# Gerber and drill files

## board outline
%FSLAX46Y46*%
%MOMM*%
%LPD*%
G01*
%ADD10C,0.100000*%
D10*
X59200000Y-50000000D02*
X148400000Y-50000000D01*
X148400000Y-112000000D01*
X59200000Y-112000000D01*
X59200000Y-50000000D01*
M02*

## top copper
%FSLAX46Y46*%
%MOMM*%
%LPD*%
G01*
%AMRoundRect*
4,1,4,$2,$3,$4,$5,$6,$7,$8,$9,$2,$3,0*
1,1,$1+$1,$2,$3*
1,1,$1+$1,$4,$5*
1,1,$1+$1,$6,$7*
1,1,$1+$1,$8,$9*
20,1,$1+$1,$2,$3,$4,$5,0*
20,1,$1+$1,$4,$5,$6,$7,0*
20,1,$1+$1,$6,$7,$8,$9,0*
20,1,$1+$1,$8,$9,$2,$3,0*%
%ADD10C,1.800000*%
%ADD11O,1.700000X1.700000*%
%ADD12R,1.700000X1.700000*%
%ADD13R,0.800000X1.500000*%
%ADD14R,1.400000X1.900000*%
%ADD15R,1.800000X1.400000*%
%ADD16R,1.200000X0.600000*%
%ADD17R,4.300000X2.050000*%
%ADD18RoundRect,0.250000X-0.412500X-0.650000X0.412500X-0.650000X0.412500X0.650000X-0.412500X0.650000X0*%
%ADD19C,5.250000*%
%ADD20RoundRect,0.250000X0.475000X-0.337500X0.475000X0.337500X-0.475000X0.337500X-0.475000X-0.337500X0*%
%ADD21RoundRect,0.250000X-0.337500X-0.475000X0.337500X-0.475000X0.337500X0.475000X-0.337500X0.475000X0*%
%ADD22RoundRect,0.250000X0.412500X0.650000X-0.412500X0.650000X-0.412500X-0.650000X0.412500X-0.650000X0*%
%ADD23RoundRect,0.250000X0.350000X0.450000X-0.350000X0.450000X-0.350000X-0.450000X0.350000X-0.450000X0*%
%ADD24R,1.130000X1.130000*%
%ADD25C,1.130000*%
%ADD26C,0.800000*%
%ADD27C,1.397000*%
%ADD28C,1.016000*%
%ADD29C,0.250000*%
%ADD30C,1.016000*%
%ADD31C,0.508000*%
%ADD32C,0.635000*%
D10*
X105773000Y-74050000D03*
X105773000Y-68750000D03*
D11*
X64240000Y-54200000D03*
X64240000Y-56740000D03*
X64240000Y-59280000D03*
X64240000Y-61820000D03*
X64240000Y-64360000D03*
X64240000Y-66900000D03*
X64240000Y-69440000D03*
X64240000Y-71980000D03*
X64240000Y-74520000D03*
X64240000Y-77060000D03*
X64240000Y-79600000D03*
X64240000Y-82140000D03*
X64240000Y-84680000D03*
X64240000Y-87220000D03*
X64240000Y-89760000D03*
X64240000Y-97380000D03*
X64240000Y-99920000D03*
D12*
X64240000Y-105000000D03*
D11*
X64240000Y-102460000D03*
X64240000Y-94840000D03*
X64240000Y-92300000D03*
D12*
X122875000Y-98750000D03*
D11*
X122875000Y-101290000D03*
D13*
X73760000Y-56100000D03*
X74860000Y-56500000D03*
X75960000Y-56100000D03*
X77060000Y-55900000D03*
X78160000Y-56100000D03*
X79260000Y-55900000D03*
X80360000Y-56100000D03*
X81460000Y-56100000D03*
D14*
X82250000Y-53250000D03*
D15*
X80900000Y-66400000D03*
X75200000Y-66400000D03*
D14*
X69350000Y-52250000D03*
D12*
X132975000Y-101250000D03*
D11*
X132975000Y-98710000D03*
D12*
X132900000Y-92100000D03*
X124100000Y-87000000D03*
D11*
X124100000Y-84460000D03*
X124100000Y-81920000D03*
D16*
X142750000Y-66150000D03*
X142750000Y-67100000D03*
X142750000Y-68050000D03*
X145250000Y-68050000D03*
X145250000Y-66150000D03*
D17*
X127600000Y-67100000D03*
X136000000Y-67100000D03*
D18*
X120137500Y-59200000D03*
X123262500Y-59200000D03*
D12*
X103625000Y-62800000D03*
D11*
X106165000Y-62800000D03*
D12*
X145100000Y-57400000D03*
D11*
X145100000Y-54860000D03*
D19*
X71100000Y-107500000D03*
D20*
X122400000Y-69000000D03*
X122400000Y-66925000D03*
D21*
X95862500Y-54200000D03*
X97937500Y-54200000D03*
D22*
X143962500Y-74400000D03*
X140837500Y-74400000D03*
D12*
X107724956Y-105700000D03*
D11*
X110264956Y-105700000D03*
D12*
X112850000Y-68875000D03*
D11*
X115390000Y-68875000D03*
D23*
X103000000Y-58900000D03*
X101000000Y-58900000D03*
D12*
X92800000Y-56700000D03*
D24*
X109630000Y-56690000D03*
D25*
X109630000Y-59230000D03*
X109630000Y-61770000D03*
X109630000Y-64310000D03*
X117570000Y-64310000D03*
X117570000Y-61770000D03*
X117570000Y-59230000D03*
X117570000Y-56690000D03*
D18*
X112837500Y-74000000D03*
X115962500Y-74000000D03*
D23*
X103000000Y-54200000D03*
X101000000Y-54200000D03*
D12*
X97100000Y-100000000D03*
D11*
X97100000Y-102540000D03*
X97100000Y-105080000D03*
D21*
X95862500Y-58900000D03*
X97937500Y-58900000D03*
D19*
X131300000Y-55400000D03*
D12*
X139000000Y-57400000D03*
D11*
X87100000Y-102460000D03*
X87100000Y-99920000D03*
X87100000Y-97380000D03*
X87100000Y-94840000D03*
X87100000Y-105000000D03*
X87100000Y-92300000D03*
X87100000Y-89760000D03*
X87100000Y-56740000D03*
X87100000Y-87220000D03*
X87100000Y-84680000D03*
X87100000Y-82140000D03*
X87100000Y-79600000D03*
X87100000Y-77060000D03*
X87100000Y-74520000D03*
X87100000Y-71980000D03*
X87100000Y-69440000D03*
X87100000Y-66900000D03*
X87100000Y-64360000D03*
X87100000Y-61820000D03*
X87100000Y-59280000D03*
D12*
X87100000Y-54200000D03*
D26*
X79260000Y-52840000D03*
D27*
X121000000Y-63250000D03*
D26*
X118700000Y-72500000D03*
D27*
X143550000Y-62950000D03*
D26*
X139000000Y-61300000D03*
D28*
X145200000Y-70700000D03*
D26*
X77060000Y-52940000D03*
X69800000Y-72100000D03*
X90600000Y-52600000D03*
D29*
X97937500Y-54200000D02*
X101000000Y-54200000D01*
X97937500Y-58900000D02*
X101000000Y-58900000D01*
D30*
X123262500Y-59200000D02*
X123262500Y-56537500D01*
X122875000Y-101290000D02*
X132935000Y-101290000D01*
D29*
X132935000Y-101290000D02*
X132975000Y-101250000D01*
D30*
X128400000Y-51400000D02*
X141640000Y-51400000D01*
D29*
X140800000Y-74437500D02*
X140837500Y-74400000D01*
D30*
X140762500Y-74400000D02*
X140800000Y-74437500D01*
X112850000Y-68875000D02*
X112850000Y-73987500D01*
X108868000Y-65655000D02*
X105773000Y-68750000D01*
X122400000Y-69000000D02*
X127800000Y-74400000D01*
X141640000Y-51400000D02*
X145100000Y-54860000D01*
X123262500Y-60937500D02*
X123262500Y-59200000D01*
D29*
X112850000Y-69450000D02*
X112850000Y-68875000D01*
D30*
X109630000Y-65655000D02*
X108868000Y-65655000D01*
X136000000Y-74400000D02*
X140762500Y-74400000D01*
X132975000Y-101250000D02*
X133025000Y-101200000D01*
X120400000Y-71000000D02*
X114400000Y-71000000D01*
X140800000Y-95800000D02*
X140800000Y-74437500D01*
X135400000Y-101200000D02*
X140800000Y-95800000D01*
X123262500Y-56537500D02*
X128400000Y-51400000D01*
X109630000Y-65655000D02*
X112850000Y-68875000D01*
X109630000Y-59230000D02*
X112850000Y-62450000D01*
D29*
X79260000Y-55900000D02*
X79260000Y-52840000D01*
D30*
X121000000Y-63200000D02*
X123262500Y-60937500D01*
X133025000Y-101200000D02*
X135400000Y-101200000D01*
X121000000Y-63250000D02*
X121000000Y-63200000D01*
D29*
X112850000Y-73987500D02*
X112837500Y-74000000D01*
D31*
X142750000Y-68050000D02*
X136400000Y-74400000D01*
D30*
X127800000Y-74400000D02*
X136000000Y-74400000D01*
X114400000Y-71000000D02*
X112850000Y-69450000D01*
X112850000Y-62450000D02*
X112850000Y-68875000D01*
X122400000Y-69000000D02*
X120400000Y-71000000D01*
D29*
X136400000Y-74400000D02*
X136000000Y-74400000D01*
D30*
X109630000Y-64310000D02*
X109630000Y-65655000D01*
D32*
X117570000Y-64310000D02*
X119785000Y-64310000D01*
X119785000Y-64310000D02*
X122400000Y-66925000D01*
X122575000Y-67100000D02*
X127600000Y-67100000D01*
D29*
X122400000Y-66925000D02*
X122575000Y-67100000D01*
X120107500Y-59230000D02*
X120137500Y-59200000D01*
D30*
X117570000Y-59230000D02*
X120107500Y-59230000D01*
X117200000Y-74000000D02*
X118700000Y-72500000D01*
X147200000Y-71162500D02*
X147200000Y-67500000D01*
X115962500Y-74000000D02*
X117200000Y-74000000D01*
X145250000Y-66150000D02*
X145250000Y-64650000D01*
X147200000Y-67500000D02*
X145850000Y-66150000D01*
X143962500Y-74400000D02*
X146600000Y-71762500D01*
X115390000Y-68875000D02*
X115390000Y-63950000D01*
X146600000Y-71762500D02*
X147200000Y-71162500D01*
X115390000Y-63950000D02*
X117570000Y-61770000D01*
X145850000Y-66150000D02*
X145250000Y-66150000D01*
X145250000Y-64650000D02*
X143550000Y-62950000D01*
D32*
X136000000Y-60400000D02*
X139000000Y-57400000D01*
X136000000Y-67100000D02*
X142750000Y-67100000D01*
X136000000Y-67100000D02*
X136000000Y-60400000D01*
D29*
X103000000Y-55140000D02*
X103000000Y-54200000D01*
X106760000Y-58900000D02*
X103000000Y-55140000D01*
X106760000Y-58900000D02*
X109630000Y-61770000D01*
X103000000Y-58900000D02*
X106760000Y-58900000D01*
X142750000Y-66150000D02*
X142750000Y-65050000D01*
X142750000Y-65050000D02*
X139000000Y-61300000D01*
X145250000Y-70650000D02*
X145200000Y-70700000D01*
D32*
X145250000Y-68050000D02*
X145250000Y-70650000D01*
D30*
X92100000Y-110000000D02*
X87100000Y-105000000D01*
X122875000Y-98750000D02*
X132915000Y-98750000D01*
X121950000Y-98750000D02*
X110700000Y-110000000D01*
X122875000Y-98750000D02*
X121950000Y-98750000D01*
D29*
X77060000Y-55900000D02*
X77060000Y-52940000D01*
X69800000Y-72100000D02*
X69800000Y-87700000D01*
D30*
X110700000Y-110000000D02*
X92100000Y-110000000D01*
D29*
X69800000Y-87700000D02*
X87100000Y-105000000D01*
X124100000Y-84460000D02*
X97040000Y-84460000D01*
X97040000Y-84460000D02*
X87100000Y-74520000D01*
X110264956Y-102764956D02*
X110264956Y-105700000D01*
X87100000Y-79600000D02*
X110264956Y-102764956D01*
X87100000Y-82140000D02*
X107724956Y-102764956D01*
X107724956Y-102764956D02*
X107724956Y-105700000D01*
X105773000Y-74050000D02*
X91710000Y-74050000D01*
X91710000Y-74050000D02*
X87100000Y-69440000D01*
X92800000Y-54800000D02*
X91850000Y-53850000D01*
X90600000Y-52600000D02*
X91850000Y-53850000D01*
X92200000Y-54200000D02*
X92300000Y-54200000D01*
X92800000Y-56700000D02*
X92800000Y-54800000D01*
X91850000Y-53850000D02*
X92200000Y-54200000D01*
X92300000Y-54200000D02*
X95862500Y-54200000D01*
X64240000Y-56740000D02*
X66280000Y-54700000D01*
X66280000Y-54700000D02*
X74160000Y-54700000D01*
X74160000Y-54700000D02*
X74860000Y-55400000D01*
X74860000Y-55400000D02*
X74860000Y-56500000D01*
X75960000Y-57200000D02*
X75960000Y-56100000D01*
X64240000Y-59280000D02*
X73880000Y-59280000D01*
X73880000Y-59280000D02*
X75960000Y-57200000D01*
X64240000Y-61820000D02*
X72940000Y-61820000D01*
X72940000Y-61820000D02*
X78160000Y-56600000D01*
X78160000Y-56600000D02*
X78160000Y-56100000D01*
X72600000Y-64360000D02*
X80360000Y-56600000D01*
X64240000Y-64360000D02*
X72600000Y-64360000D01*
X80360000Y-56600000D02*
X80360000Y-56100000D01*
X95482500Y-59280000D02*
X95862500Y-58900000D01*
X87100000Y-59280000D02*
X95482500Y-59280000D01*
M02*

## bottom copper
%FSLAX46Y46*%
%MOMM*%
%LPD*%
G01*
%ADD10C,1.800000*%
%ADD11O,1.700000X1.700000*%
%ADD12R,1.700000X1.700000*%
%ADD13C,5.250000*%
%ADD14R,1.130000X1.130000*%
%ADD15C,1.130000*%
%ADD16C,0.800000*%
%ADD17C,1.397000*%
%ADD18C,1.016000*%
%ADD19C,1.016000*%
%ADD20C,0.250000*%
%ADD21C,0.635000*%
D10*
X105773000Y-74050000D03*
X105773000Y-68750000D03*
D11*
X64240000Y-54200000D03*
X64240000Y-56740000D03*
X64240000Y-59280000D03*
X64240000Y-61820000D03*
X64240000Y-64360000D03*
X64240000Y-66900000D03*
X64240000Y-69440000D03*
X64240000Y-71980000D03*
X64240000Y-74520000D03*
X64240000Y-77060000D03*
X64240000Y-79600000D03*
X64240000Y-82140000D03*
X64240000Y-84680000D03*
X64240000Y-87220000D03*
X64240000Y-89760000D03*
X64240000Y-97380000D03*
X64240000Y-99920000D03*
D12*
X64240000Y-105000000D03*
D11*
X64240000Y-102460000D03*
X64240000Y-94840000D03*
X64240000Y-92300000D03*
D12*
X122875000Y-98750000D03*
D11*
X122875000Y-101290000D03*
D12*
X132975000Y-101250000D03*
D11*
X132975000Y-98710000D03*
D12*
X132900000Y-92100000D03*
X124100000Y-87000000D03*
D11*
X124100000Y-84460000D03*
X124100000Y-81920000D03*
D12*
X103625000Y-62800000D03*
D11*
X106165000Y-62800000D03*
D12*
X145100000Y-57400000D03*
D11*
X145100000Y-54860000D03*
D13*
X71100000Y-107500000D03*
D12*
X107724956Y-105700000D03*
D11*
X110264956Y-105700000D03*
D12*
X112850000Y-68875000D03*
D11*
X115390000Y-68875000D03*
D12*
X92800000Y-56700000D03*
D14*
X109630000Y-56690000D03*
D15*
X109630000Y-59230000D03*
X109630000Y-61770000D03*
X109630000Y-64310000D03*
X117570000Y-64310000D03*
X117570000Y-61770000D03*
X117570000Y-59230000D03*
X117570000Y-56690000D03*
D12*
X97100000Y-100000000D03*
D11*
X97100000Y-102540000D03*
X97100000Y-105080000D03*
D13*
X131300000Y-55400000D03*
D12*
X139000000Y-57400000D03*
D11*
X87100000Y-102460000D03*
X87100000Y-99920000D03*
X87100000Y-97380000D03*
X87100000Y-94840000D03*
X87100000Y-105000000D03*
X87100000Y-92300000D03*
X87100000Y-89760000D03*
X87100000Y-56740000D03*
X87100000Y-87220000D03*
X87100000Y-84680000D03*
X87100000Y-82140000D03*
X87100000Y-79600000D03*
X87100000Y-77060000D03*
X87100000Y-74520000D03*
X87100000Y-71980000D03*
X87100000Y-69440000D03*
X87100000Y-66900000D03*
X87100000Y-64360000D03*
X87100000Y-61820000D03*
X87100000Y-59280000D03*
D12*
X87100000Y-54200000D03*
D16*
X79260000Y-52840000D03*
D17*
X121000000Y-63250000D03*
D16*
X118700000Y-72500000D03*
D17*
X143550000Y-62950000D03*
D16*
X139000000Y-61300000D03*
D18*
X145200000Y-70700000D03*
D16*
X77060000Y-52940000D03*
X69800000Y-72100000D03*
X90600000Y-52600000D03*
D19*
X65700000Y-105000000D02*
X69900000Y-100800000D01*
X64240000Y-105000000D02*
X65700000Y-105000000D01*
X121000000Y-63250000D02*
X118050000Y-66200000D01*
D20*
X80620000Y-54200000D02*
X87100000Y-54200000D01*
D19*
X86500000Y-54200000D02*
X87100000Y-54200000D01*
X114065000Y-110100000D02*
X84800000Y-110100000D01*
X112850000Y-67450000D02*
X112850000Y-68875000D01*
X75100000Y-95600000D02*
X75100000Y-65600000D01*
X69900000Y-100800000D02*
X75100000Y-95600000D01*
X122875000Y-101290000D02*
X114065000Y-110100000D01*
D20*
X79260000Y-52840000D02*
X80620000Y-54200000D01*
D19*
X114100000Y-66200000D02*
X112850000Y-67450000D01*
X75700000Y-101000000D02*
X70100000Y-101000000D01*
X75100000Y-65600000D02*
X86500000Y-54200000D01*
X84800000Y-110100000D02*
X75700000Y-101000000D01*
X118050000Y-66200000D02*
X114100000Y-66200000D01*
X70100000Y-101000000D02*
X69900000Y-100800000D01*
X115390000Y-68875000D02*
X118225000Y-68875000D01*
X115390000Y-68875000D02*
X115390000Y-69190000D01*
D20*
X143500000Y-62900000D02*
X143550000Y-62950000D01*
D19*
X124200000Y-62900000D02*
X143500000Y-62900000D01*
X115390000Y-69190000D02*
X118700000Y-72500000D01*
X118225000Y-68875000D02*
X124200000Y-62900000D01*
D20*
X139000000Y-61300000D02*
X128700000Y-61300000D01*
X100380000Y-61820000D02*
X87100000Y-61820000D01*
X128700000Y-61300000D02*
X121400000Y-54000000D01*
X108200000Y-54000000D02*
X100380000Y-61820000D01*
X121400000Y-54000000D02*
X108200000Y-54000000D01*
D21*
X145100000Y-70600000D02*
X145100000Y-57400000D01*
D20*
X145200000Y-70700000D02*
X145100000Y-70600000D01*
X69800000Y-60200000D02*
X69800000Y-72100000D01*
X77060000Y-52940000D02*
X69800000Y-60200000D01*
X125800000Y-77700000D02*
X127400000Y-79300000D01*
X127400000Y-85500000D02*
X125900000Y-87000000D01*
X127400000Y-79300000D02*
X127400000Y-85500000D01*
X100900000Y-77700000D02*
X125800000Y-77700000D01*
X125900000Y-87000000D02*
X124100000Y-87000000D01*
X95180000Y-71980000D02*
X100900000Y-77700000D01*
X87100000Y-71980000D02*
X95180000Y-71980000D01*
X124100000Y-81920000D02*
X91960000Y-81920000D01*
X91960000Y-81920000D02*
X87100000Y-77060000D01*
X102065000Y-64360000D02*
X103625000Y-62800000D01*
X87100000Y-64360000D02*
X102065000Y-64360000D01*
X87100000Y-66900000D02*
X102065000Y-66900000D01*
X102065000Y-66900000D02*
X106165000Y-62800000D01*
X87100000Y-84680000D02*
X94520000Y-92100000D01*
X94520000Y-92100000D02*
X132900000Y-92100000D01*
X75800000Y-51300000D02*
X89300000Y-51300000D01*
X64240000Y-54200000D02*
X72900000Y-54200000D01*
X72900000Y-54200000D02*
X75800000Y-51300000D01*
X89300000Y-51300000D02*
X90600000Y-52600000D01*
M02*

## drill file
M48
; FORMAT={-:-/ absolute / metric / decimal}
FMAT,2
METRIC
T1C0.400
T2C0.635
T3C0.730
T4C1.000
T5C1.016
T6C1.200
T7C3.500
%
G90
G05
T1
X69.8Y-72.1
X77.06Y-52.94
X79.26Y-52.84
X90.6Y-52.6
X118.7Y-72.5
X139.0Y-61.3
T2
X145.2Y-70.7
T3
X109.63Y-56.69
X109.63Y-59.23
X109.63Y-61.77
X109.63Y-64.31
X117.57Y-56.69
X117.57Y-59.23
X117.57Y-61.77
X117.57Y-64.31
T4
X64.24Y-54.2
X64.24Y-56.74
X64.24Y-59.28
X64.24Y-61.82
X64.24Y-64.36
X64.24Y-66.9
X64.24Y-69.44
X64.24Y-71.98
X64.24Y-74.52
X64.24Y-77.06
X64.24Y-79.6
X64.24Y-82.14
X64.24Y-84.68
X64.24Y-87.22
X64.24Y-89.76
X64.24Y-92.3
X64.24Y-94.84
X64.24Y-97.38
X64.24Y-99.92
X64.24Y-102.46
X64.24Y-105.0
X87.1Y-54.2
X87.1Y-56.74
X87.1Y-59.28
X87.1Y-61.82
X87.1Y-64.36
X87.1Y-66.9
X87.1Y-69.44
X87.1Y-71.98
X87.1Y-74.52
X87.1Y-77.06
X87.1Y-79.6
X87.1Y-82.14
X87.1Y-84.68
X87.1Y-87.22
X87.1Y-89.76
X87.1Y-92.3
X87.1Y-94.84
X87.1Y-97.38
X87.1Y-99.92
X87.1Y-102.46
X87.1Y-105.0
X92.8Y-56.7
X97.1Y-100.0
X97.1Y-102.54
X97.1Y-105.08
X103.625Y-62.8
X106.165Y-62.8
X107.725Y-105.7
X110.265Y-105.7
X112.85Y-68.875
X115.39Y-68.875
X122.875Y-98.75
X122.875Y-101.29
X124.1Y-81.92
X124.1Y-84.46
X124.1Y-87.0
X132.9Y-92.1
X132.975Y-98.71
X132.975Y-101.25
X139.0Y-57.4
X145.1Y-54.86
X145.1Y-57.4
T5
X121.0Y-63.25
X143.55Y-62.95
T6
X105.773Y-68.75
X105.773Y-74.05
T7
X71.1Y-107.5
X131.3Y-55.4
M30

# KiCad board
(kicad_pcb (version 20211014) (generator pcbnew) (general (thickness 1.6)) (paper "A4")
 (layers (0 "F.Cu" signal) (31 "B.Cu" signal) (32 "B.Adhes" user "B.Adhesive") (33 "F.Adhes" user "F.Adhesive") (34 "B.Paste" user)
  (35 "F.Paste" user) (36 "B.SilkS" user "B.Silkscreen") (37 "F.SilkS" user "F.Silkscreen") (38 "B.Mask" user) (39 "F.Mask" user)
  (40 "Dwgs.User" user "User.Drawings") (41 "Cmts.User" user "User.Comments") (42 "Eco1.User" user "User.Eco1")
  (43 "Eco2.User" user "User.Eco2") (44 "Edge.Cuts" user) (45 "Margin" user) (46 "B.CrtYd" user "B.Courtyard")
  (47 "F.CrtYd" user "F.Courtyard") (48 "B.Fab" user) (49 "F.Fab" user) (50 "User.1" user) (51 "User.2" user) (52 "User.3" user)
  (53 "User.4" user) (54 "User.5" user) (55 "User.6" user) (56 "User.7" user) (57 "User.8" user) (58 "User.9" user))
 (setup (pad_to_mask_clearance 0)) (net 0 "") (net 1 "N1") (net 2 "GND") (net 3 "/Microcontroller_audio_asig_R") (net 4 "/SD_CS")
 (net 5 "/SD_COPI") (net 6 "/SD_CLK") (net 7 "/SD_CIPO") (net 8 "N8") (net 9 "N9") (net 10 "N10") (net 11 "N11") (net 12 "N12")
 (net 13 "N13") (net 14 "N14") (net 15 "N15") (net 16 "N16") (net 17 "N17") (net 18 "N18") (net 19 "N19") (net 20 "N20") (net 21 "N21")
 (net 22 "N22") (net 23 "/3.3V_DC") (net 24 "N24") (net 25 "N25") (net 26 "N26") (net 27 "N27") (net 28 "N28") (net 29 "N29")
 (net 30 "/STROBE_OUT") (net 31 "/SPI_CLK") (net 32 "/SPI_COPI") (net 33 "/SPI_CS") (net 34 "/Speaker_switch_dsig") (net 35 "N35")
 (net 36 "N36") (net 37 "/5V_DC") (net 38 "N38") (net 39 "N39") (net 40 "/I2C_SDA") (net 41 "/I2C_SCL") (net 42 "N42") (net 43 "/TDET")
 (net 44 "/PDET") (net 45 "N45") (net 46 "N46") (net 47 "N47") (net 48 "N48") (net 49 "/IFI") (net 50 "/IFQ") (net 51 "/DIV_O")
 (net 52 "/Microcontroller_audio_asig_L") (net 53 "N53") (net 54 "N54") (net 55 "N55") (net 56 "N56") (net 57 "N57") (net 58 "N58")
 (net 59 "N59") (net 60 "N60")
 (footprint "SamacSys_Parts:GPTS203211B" (layer "F.Cu") (at 105.854 71.4)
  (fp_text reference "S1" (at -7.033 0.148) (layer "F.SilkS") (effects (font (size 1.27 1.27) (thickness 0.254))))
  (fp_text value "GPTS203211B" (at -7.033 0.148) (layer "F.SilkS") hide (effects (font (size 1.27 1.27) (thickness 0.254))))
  (pad "1" thru_hole circle locked (at -0.081 2.65) (size 1.8 1.8) (drill 1.2) (layers *.Cu *.Mask) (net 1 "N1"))
  (pad "2" thru_hole circle locked (at -0.081 -2.65) (size 1.8 1.8) (drill 1.2) (layers *.Cu *.Mask) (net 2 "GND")))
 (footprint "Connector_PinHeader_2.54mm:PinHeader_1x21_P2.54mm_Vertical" (layer "F.Cu") (at 64.24 105 180)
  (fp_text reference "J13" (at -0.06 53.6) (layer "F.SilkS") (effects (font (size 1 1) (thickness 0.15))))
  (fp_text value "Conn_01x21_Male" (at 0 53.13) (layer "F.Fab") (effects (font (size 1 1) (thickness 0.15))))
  (pad "18" thru_hole oval (at 0 50.8 180) (size 1.7 1.7) (drill 1) (layers *.Cu *.Mask) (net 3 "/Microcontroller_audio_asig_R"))
  (pad "19" thru_hole oval (at 0 48.26 180) (size 1.7 1.7) (drill 1) (layers *.Cu *.Mask) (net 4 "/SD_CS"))
  (pad "20" thru_hole oval (at 0 45.72 180) (size 1.7 1.7) (drill 1) (layers *.Cu *.Mask) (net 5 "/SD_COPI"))
  (pad "21" thru_hole oval (at 0 43.18 180) (size 1.7 1.7) (drill 1) (layers *.Cu *.Mask) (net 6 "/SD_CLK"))
  (pad "26" thru_hole oval (at 0 40.64 180) (size 1.7 1.7) (drill 1) (layers *.Cu *.Mask) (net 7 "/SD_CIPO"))
  (pad "33" thru_hole oval (at 0 38.1 180) (size 1.7 1.7) (drill 1) (layers *.Cu *.Mask) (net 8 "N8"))
  (pad "34" thru_hole oval (at 0 35.56 180) (size 1.7 1.7) (drill 1) (layers *.Cu *.Mask) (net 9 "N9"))
  (pad "35" thru_hole oval (at 0 33.02 180) (size 1.7 1.7) (drill 1) (layers *.Cu *.Mask) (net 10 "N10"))
  (pad "36" thru_hole oval (at 0 30.48 180) (size 1.7 1.7) (drill 1) (layers *.Cu *.Mask) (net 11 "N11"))
  (pad "37" thru_hole oval (at 0 27.94 180) (size 1.7 1.7) (drill 1) (layers *.Cu *.Mask) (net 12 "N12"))
  (pad "38" thru_hole oval (at 0 25.4 180) (size 1.7 1.7) (drill 1) (layers *.Cu *.Mask) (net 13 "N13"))
  (pad "39" thru_hole oval (at 0 22.86 180) (size 1.7 1.7) (drill 1) (layers *.Cu *.Mask) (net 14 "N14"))
  (pad "40" thru_hole oval (at 0 20.32 180) (size 1.7 1.7) (drill 1) (layers *.Cu *.Mask) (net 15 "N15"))
  (pad "41" thru_hole oval (at 0 17.78 180) (size 1.7 1.7) (drill 1) (layers *.Cu *.Mask) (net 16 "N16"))
  (pad "42" thru_hole oval (at 0 15.24 180) (size 1.7 1.7) (drill 1) (layers *.Cu *.Mask) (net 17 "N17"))
  (pad "45" thru_hole oval (at 0 7.62 180) (size 1.7 1.7) (drill 1) (layers *.Cu *.Mask) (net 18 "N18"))
  (pad "46" thru_hole oval (at 0 5.08 180) (size 1.7 1.7) (drill 1) (layers *.Cu *.Mask) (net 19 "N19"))
  (pad "G" thru_hole rect (at 0 0 180) (size 1.7 1.7) (drill 1) (layers *.Cu *.Mask) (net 2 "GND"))
  (pad "RST" thru_hole oval (at 0 2.54 180) (size 1.7 1.7) (drill 1) (layers *.Cu *.Mask) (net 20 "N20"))
  (pad "RX" thru_hole oval (at 0 10.16 180) (size 1.7 1.7) (drill 1) (layers *.Cu *.Mask) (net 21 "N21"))
  (pad "TX" thru_hole oval (at 0 12.7 270) (size 1.7 1.7) (drill 1) (layers *.Cu *.Mask) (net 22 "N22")))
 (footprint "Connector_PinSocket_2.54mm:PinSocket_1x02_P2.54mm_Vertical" (layer "F.Cu") (at 122.875 98.75)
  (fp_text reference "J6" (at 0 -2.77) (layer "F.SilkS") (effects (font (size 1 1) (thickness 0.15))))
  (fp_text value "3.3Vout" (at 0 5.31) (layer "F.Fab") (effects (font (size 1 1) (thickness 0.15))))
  (pad "1" thru_hole rect (at 0 0) (size 1.7 1.7) (drill 1) (layers *.Cu *.Mask) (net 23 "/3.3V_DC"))
  (pad "2" thru_hole oval (at 0 2.54) (size 1.7 1.7) (drill 1) (layers *.Cu *.Mask) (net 2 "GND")))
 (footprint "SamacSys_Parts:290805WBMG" (layer "F.Cu") (at 75.8 59.2)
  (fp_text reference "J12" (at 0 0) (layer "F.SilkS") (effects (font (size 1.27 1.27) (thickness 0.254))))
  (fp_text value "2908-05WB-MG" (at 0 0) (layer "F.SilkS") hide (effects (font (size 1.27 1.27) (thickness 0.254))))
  (pad "1" smd rect locked (at -2.04 -3.1) (size 0.8 1.5) (layers "F.Cu" "F.Paste" "F.Mask") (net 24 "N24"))
  (pad "2" smd rect locked (at -0.94 -2.7) (size 0.8 1.5) (layers "F.Cu" "F.Paste" "F.Mask") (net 4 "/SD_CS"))
  (pad "3" smd rect locked (at 0.16 -3.1) (size 0.8 1.5) (layers "F.Cu" "F.Paste" "F.Mask") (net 5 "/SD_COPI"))
  (pad "4" smd rect locked (at 1.26 -3.3) (size 0.8 1.5) (layers "F.Cu" "F.Paste" "F.Mask") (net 23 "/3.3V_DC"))
  (pad "5" smd rect locked (at 2.36 -3.1) (size 0.8 1.5) (layers "F.Cu" "F.Paste" "F.Mask") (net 6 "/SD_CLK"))
  (pad "6" smd rect locked (at 3.46 -3.3) (size 0.8 1.5) (layers "F.Cu" "F.Paste" "F.Mask") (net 2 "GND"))
  (pad "7" smd rect locked (at 4.56 -3.1) (size 0.8 1.5) (layers "F.Cu" "F.Paste" "F.Mask") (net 7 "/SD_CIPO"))
  (pad "8" smd rect locked (at 5.66 -3.1) (size 0.8 1.5) (layers "F.Cu" "F.Paste" "F.Mask") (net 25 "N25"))
  (pad "MP1" smd rect locked (at 6.45 -5.95) (size 1.4 1.9) (layers "F.Cu" "F.Paste" "F.Mask") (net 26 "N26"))
  (pad "MP2" smd rect locked (at 5.1 7.2 90) (size 1.4 1.8) (layers "F.Cu" "F.Paste" "F.Mask") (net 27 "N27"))
  (pad "MP3" smd rect locked (at -0.6 7.2 90) (size 1.4 1.8) (layers "F.Cu" "F.Paste" "F.Mask") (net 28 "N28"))
  (pad "MP4" smd rect locked (at -6.45 -6.95) (size 1.4 1.9) (layers "F.Cu" "F.Paste" "F.Mask") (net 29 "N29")))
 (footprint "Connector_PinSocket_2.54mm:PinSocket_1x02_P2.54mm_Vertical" (layer "F.Cu") (at 132.975 101.25 180)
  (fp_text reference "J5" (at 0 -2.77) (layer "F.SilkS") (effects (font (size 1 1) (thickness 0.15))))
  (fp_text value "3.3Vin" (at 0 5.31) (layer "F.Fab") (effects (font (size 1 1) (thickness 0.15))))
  (pad "1" thru_hole rect (at 0 0 180) (size 1.7 1.7) (drill 1) (layers *.Cu *.Mask) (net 2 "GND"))
  (pad "2" thru_hole oval (at 0 2.54 180) (size 1.7 1.7) (drill 1) (layers *.Cu *.Mask) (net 23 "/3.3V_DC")))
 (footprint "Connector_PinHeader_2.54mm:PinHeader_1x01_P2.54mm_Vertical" (layer "F.Cu") (at 132.9 92.1)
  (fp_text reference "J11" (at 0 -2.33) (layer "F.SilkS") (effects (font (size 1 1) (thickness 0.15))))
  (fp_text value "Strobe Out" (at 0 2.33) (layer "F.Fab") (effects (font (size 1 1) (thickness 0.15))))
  (pad "1" thru_hole rect (at 0 0) (size 1.7 1.7) (drill 1) (layers *.Cu *.Mask) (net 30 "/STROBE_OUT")))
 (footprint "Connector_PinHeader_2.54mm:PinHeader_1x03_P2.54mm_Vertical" (layer "F.Cu") (at 124.1 87 180)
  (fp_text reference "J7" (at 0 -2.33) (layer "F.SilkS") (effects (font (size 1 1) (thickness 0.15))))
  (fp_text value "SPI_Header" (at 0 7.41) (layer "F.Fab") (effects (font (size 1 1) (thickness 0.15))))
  (pad "1" thru_hole rect (at 0 0 180) (size 1.7 1.7) (drill 1) (layers *.Cu *.Mask) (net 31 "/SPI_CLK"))
  (pad "2" thru_hole oval (at 0 2.54 180) (size 1.7 1.7) (drill 1) (layers *.Cu *.Mask) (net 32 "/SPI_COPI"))
  (pad "3" thru_hole oval (at 0 5.08 180) (size 1.7 1.7) (drill 1) (layers *.Cu *.Mask) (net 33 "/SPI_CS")))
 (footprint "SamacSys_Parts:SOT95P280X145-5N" (layer "F.Cu") (at 144 67.1)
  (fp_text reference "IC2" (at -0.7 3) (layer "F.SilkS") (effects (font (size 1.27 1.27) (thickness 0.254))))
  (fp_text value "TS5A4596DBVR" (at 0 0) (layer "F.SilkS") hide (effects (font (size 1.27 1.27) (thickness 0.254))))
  (pad "1" smd rect locked (at -1.25 -0.95 90) (size 0.6 1.2) (layers "F.Cu" "F.Paste" "F.Mask") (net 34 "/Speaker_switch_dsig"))
  (pad "2" smd rect locked (at -1.25 0 90) (size 0.6 1.2) (layers "F.Cu" "F.Paste" "F.Mask") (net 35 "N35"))
  (pad "3" smd rect locked (at -1.25 0.95 90) (size 0.6 1.2) (layers "F.Cu" "F.Paste" "F.Mask") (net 2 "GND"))
  (pad "4" smd rect locked (at 1.25 0.95 90) (size 0.6 1.2) (layers "F.Cu" "F.Paste" "F.Mask") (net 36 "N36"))
  (pad "5" smd rect locked (at 1.25 -0.95 90) (size 0.6 1.2) (layers "F.Cu" "F.Paste" "F.Mask") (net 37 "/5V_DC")))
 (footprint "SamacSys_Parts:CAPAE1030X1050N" (layer "F.Cu") (at 131.8 67.1)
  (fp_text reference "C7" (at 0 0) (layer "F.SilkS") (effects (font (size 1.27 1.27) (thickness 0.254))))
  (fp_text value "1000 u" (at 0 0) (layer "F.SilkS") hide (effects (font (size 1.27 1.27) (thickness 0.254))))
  (pad "1" smd rect locked (at -4.2 0 90) (size 2.05 4.3) (layers "F.Cu" "F.Paste" "F.Mask") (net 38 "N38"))
  (pad "2" smd rect locked (at 4.2 0 90) (size 2.05 4.3) (layers "F.Cu" "F.Paste" "F.Mask") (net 35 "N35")))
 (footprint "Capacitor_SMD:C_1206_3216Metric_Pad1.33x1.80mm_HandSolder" (layer "F.Cu") (at 121.7 59.2)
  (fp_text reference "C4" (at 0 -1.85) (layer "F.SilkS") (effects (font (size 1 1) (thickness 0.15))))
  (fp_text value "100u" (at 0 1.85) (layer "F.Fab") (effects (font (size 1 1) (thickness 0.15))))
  (pad "1" smd roundrect (at -1.5625 0) (size 1.325 1.8) (layers "F.Cu" "F.Paste" "F.Mask") (roundrect_rratio 0.1886792453) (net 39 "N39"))
  (pad "2" smd roundrect (at 1.5625 0) (size 1.325 1.8) (layers "F.Cu" "F.Paste" "F.Mask") (roundrect_rratio 0.1886792453) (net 2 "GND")))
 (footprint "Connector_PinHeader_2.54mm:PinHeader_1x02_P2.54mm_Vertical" (layer "F.Cu") (at 103.625 62.8 90)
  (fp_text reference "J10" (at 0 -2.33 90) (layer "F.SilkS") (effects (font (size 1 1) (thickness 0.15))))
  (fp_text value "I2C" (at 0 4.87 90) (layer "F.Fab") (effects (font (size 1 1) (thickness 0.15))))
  (pad "1" thru_hole rect (at 0 0 90) (size 1.7 1.7) (drill 1) (layers *.Cu *.Mask) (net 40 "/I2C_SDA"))
  (pad "2" thru_hole oval (at 0 2.54 90) (size 1.7 1.7) (drill 1) (layers *.Cu *.Mask) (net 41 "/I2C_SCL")))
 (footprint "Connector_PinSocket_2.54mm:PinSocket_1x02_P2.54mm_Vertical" (layer "F.Cu") (at 145.1 57.4 180)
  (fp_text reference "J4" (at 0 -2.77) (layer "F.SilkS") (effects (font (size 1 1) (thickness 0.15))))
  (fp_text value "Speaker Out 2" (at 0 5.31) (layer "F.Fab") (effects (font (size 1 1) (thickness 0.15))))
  (pad "1" thru_hole rect (at 0 0 180) (size 1.7 1.7) (drill 1) (layers *.Cu *.Mask) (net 36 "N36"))
  (pad "2" thru_hole oval (at 0 2.54 180) (size 1.7 1.7) (drill 1) (layers *.Cu *.Mask) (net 2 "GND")))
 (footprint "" (layer "F.Cu") (at 71.1 107.5)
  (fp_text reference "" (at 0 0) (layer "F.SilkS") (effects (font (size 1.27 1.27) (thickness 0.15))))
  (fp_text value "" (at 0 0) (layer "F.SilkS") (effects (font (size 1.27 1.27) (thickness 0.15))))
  (pad "MH1" thru_hole circle (at 0 0 90) (size 5.25 5.25) (drill 3.5) (layers *.Cu *.Mask)))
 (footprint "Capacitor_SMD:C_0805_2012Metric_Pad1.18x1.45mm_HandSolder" (layer "F.Cu") (at 122.4 67.9625 90)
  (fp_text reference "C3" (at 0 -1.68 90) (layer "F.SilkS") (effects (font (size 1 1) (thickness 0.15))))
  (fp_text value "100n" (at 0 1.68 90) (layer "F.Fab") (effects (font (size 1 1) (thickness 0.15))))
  (pad "1" smd roundrect (at -1.0375 0 90) (size 1.175 1.45) (layers "F.Cu" "F.Paste" "F.Mask") (roundrect_rratio 0.2127659574)
   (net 2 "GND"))
  (pad "2" smd roundrect (at 1.0375 0 90) (size 1.175 1.45) (layers "F.Cu" "F.Paste" "F.Mask") (roundrect_rratio 0.2127659574)
   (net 38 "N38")))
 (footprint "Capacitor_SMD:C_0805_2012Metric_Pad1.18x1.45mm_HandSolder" (layer "F.Cu") (at 96.9 54.2)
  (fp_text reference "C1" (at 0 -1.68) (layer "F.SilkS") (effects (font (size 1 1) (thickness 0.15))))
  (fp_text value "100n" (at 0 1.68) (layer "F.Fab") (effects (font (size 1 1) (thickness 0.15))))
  (pad "1" smd roundrect (at -1.0375 0) (size 1.175 1.45) (layers "F.Cu" "F.Paste" "F.Mask") (roundrect_rratio 0.2127659574)
   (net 3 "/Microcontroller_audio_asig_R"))
  (pad "2" smd roundrect (at 1.0375 0) (size 1.175 1.45) (layers "F.Cu" "F.Paste" "F.Mask") (roundrect_rratio 0.2127659574) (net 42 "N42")))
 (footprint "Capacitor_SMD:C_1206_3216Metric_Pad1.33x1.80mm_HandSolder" (layer "F.Cu") (at 142.4 74.4 180)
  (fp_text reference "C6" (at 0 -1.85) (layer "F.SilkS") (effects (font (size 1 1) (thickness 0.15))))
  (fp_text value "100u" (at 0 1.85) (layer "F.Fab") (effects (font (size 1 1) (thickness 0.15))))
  (pad "1" smd roundrect (at -1.5625 0 180) (size 1.325 1.8) (layers "F.Cu" "F.Paste" "F.Mask") (roundrect_rratio 0.1886792453)
   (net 37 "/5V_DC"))
  (pad "2" smd roundrect (at 1.5625 0 180) (size 1.325 1.8) (layers "F.Cu" "F.Paste" "F.Mask") (roundrect_rratio 0.1886792453) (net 2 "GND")))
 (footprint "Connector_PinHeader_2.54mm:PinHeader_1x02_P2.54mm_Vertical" (layer "F.Cu") (at 107.724956 105.7 90)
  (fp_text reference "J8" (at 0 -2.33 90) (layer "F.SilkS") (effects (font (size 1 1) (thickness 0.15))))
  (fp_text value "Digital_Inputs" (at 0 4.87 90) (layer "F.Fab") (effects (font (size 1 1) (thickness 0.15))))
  (pad "1" thru_hole rect (at 0 0 90) (size 1.7 1.7) (drill 1) (layers *.Cu *.Mask) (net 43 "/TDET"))
  (pad "2" thru_hole oval (at 0 2.54 90) (size 1.7 1.7) (drill 1) (layers *.Cu *.Mask) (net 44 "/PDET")))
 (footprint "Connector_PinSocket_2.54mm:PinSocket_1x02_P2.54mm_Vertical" (layer "F.Cu") (at 112.85 68.875 90)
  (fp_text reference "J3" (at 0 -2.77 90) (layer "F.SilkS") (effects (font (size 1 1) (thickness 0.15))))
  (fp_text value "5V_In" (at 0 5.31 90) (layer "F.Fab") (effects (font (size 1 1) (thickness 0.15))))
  (pad "1" thru_hole rect (at 0 0 90) (size 1.7 1.7) (drill 1) (layers *.Cu *.Mask) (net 2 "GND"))
  (pad "2" thru_hole oval (at 0 2.54 90) (size 1.7 1.7) (drill 1) (layers *.Cu *.Mask) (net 37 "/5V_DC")))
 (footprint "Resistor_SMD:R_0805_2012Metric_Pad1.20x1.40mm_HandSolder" (layer "F.Cu") (at 102 58.9 180)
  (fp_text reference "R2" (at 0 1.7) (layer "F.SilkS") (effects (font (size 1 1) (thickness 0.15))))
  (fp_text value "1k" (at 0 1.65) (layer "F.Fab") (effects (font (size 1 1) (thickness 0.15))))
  (pad "1" smd roundrect (at -1 0 180) (size 1.2 1.4) (layers "F.Cu" "F.Paste" "F.Mask") (roundrect_rratio 0.2083333333) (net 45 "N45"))
  (pad "2" smd roundrect (at 1 0 180) (size 1.2 1.4) (layers "F.Cu" "F.Paste" "F.Mask") (roundrect_rratio 0.2083333333) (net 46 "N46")))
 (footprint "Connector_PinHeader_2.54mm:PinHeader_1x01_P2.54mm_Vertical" (layer "F.Cu") (at 92.8 56.7)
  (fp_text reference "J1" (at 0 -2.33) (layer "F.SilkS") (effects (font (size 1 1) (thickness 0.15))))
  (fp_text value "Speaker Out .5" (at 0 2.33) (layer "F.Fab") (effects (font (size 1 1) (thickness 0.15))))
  (pad "1" thru_hole rect (at 0 0) (size 1.7 1.7) (drill 1) (layers *.Cu *.Mask) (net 3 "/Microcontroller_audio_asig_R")))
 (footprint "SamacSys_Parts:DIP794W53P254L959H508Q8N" (layer "F.Cu") (at 113.6 60.5)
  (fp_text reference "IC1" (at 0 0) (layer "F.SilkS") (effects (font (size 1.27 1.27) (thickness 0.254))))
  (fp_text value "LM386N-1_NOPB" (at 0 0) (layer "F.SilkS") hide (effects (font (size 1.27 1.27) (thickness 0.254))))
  (pad "1" thru_hole rect locked (at -3.97 -3.81) (size 1.13 1.13) (drill 0.73) (layers *.Cu *.Mask) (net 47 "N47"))
  (pad "2" thru_hole circle locked (at -3.97 -1.27) (size 1.13 1.13) (drill 0.73) (layers *.Cu *.Mask) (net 2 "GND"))
  (pad "3" thru_hole circle locked (at -3.97 1.27) (size 1.13 1.13) (drill 0.73) (layers *.Cu *.Mask) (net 45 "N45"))
  (pad "4" thru_hole circle locked (at -3.97 3.81) (size 1.13 1.13) (drill 0.73) (layers *.Cu *.Mask) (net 2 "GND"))
  (pad "5" thru_hole circle locked (at 3.97 3.81) (size 1.13 1.13) (drill 0.73) (layers *.Cu *.Mask) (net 38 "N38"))
  (pad "6" thru_hole circle locked (at 3.97 1.27) (size 1.13 1.13) (drill 0.73) (layers *.Cu *.Mask) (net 37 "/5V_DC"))
  (pad "7" thru_hole circle locked (at 3.97 -1.27) (size 1.13 1.13) (drill 0.73) (layers *.Cu *.Mask) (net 39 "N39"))
  (pad "8" thru_hole circle locked (at 3.97 -3.81) (size 1.13 1.13) (drill 0.73) (layers *.Cu *.Mask) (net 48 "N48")))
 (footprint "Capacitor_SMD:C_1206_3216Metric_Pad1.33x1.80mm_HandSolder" (layer "F.Cu") (at 114.4 74)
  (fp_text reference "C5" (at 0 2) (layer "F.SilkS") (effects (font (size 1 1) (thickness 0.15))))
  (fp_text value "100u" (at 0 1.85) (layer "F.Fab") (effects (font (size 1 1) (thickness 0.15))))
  (pad "1" smd roundrect (at -1.5625 0) (size 1.325 1.8) (layers "F.Cu" "F.Paste" "F.Mask") (roundrect_rratio 0.1886792453) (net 2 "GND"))
  (pad "2" smd roundrect (at 1.5625 0) (size 1.325 1.8) (layers "F.Cu" "F.Paste" "F.Mask") (roundrect_rratio 0.1886792453) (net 37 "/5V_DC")))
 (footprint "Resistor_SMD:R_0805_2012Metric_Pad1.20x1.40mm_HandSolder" (layer "F.Cu") (at 102 54.2 180)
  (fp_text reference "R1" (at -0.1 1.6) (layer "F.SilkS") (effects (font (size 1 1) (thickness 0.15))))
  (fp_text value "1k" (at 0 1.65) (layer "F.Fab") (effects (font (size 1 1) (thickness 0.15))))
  (pad "1" smd roundrect (at -1 0 180) (size 1.2 1.4) (layers "F.Cu" "F.Paste" "F.Mask") (roundrect_rratio 0.2083333333) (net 45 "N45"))
  (pad "2" smd roundrect (at 1 0 180) (size 1.2 1.4) (layers "F.Cu" "F.Paste" "F.Mask") (roundrect_rratio 0.2083333333) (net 42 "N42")))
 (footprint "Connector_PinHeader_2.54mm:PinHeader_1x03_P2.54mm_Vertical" (layer "F.Cu") (at 97.1 100)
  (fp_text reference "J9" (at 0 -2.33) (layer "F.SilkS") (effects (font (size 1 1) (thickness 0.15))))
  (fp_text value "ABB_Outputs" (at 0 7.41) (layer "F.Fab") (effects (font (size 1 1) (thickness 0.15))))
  (pad "1" thru_hole rect (at 0 0) (size 1.7 1.7) (drill 1) (layers *.Cu *.Mask) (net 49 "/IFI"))
  (pad "2" thru_hole oval (at 0 2.54) (size 1.7 1.7) (drill 1) (layers *.Cu *.Mask) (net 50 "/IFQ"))
  (pad "3" thru_hole oval (at 0 5.08) (size 1.7 1.7) (drill 1) (layers *.Cu *.Mask) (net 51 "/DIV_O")))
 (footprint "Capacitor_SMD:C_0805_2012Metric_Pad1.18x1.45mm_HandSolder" (layer "F.Cu") (at 96.9 58.9)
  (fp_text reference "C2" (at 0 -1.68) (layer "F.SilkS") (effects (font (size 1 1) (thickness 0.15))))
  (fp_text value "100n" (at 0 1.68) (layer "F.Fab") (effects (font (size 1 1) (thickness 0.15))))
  (pad "1" smd roundrect (at -1.0375 0) (size 1.175 1.45) (layers "F.Cu" "F.Paste" "F.Mask") (roundrect_rratio 0.2127659574)
   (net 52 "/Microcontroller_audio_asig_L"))
  (pad "2" smd roundrect (at 1.0375 0) (size 1.175 1.45) (layers "F.Cu" "F.Paste" "F.Mask") (roundrect_rratio 0.2127659574) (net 46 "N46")))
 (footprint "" (layer "F.Cu") (at 131.3 55.4)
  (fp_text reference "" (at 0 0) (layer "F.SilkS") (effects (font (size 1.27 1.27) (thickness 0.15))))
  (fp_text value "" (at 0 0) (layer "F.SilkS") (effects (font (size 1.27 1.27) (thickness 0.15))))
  (pad "MH2" thru_hole circle (at 0 0 90) (size 5.25 5.25) (drill 3.5) (layers *.Cu *.Mask)))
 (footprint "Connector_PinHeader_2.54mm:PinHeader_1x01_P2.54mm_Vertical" (layer "F.Cu") (at 139 57.4)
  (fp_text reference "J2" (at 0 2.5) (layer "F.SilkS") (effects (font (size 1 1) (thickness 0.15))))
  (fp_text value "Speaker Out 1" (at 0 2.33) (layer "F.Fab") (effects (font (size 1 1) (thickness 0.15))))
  (pad "1" thru_hole rect (at 0 0) (size 1.7 1.7) (drill 1) (layers *.Cu *.Mask) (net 35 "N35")))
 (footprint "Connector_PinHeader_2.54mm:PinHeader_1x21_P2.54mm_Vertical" (layer "F.Cu") (at 87.1 54.2)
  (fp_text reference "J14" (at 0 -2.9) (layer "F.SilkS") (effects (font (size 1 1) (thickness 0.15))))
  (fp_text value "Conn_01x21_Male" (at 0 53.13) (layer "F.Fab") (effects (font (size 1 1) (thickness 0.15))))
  (pad "0" thru_hole oval (at 0 48.26) (size 1.7 1.7) (drill 1) (layers *.Cu *.Mask) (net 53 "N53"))
  (pad "1" thru_hole oval (at 0 45.72) (size 1.7 1.7) (drill 1) (layers *.Cu *.Mask) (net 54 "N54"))
  (pad "2" thru_hole oval (at 0 43.18) (size 1.7 1.7) (drill 1) (layers *.Cu *.Mask) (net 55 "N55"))
  (pad "3" thru_hole oval (at 0 40.64) (size 1.7 1.7) (drill 1) (layers *.Cu *.Mask) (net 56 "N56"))
  (pad "3V3" thru_hole oval (at 0 50.8) (size 1.7 1.7) (drill 1) (layers *.Cu *.Mask) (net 23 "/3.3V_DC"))
  (pad "4" thru_hole oval (at 0 38.1) (size 1.7 1.7) (drill 1) (layers *.Cu *.Mask) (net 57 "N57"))
  (pad "5" thru_hole oval (at 0 35.56) (size 1.7 1.7) (drill 1) (layers *.Cu *.Mask) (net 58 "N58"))
  (pad "5V" thru_hole oval (at 0 2.54) (size 1.7 1.7) (drill 1) (layers *.Cu *.Mask) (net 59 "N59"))
  (pad "6" thru_hole oval (at 0 33.02) (size 1.7 1.7) (drill 1) (layers *.Cu *.Mask) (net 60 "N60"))
  (pad "7" thru_hole oval (at 0 30.48) (size 1.7 1.7) (drill 1) (layers *.Cu *.Mask) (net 30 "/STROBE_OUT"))
  (pad "8" thru_hole oval (at 0 27.94) (size 1.7 1.7) (drill 1) (layers *.Cu *.Mask) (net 43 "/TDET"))
  (pad "9" thru_hole oval (at 0 25.4) (size 1.7 1.7) (drill 1) (layers *.Cu *.Mask) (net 44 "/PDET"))
  (pad "10" thru_hole oval (at 0 22.86) (size 1.7 1.7) (drill 1) (layers *.Cu *.Mask) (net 33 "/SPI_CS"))
  (pad "11" thru_hole oval (at 0 20.32) (size 1.7 1.7) (drill 1) (layers *.Cu *.Mask) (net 32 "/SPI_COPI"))
  (pad "12" thru_hole oval (at 0 17.78) (size 1.7 1.7) (drill 1) (layers *.Cu *.Mask) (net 31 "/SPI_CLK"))
  (pad "13" thru_hole oval (at 0 15.24) (size 1.7 1.7) (drill 1) (layers *.Cu *.Mask) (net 1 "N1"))
  (pad "14" thru_hole oval (at 0 12.7) (size 1.7 1.7) (drill 1) (layers *.Cu *.Mask) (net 41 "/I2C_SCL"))
  (pad "15" thru_hole oval (at 0 10.16) (size 1.7 1.7) (drill 1) (layers *.Cu *.Mask) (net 40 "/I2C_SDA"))
  (pad "16" thru_hole oval (at 0 7.62) (size 1.7 1.7) (drill 1) (layers *.Cu *.Mask) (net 34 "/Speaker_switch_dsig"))
  (pad "17" thru_hole oval (at 0 5.08) (size 1.7 1.7) (drill 1) (layers *.Cu *.Mask) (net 52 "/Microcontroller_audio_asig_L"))
  (pad "G" thru_hole rect (at 0 0) (size 1.7 1.7) (drill 1) (layers *.Cu *.Mask) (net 2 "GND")))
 (gr_rect (start 59.2 50) (end 148.4 112) (layer "Edge.Cuts") (width 0.1) (fill none))
 (segment (start 97.9375 54.2) (end 101 54.2) (width 0.25) (layer "F.Cu") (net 42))
 (segment (start 97.9375 58.9) (end 101 58.9) (width 0.25) (layer "F.Cu") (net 46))
 (segment (start 123.2625 59.2) (end 123.2625 56.5375) (width 1.016) (layer "F.Cu") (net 2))
 (segment (start 122.875 101.29) (end 132.935 101.29) (width 1.016) (layer "F.Cu") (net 2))
 (segment (start 132.935 101.29) (end 132.975 101.25) (width 0.25) (layer "F.Cu") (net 2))
 (segment (start 128.4 51.4) (end 141.64 51.4) (width 1.016) (layer "F.Cu") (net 2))
 (segment (start 140.8 74.4375) (end 140.8375 74.4) (width 0.25) (layer "F.Cu") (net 2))
 (segment (start 140.7625 74.4) (end 140.8 74.4375) (width 1.016) (layer "F.Cu") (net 2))
 (segment (start 112.85 68.875) (end 112.85 73.9875) (width 1.016) (layer "F.Cu") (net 2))
 (segment (start 108.868 65.655) (end 105.773 68.75) (width 1.016) (layer "F.Cu") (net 2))
 (segment (start 122.4 69) (end 127.8 74.4) (width 1.016) (layer "F.Cu") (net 2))
 (segment (start 141.64 51.4) (end 145.1 54.86) (width 1.016) (layer "F.Cu") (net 2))
 (segment (start 123.2625 60.9375) (end 123.2625 59.2) (width 1.016) (layer "F.Cu") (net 2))
 (segment (start 112.85 69.45) (end 112.85 68.875) (width 0.25) (layer "F.Cu") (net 2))
 (segment (start 109.63 65.655) (end 108.868 65.655) (width 1.016) (layer "F.Cu") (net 2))
 (segment (start 136 74.4) (end 140.7625 74.4) (width 1.016) (layer "F.Cu") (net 2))
 (segment (start 132.975 101.25) (end 133.025 101.2) (width 1.016) (layer "F.Cu") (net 2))
 (segment (start 120.4 71) (end 114.4 71) (width 1.016) (layer "F.Cu") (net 2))
 (segment (start 140.8 95.8) (end 140.8 74.4375) (width 1.016) (layer "F.Cu") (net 2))
 (segment (start 135.4 101.2) (end 140.8 95.8) (width 1.016) (layer "F.Cu") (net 2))
 (segment (start 123.2625 56.5375) (end 128.4 51.4) (width 1.016) (layer "F.Cu") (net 2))
 (segment (start 109.63 65.655) (end 112.85 68.875) (width 1.016) (layer "F.Cu") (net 2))
 (segment (start 109.63 59.23) (end 112.85 62.45) (width 1.016) (layer "F.Cu") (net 2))
 (segment (start 79.26 55.9) (end 79.26 52.84) (width 0.25) (layer "F.Cu") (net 2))
 (segment (start 121 63.2) (end 123.2625 60.9375) (width 1.016) (layer "F.Cu") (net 2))
 (segment (start 133.025 101.2) (end 135.4 101.2) (width 1.016) (layer "F.Cu") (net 2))
 (segment (start 121 63.25) (end 121 63.2) (width 1.016) (layer "F.Cu") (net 2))
 (segment (start 112.85 73.9875) (end 112.8375 74) (width 0.25) (layer "F.Cu") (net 2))
 (segment (start 142.75 68.05) (end 136.4 74.4) (width 0.508) (layer "F.Cu") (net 2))
 (segment (start 127.8 74.4) (end 136 74.4) (width 1.016) (layer "F.Cu") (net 2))
 (segment (start 114.4 71) (end 112.85 69.45) (width 1.016) (layer "F.Cu") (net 2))
 (segment (start 112.85 62.45) (end 112.85 68.875) (width 1.016) (layer "F.Cu") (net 2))
 (segment (start 122.4 69) (end 120.4 71) (width 1.016) (layer "F.Cu") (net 2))
 (segment (start 136.4 74.4) (end 136 74.4) (width 0.25) (layer "F.Cu") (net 2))
 (segment (start 109.63 64.31) (end 109.63 65.655) (width 1.016) (layer "F.Cu") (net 2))
 (via (at 79.26 52.84) (size 0.8) (drill 0.4) (layers "F.Cu" "B.Cu") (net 2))
 (via (at 121 63.25) (size 1.397) (drill 1.016) (layers "F.Cu" "B.Cu") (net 2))
 (segment (start 65.7 105) (end 69.9 100.8) (width 1.016) (layer "B.Cu") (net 2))
 (segment (start 64.24 105) (end 65.7 105) (width 1.016) (layer "B.Cu") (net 2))
 (segment (start 121 63.25) (end 118.05 66.2) (width 1.016) (layer "B.Cu") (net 2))
 (segment (start 80.62 54.2) (end 87.1 54.2) (width 0.25) (layer "B.Cu") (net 2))
 (segment (start 86.5 54.2) (end 87.1 54.2) (width 1.016) (layer "B.Cu") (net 2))
 (segment (start 114.065 110.1) (end 84.8 110.1) (width 1.016) (layer "B.Cu") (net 2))
 (segment (start 112.85 67.45) (end 112.85 68.875) (width 1.016) (layer "B.Cu") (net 2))
 (segment (start 75.1 95.6) (end 75.1 65.6) (width 1.016) (layer "B.Cu") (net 2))
 (segment (start 69.9 100.8) (end 75.1 95.6) (width 1.016) (layer "B.Cu") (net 2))
 (segment (start 122.875 101.29) (end 114.065 110.1) (width 1.016) (layer "B.Cu") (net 2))
 (segment (start 79.26 52.84) (end 80.62 54.2) (width 0.25) (layer "B.Cu") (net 2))
 (segment (start 114.1 66.2) (end 112.85 67.45) (width 1.016) (layer "B.Cu") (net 2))
 (segment (start 75.7 101) (end 70.1 101) (width 1.016) (layer "B.Cu") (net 2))
 (segment (start 75.1 65.6) (end 86.5 54.2) (width 1.016) (layer "B.Cu") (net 2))
 (segment (start 84.8 110.1) (end 75.7 101) (width 1.016) (layer "B.Cu") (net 2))
 (segment (start 118.05 66.2) (end 114.1 66.2) (width 1.016) (layer "B.Cu") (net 2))
 (segment (start 70.1 101) (end 69.9 100.8) (width 1.016) (layer "B.Cu") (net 2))
 (segment (start 117.57 64.31) (end 119.785 64.31) (width 0.635) (layer "F.Cu") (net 38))
 (segment (start 119.785 64.31) (end 122.4 66.925) (width 0.635) (layer "F.Cu") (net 38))
 (segment (start 122.575 67.1) (end 127.6 67.1) (width 0.635) (layer "F.Cu") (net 38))
 (segment (start 122.4 66.925) (end 122.575 67.1) (width 0.25) (layer "F.Cu") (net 38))
 (segment (start 120.1075 59.23) (end 120.1375 59.2) (width 0.25) (layer "F.Cu") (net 39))
 (segment (start 117.57 59.23) (end 120.1075 59.23) (width 1.016) (layer "F.Cu") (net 39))
 (segment (start 117.2 74) (end 118.7 72.5) (width 1.016) (layer "F.Cu") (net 37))
 (segment (start 147.2 71.1625) (end 147.2 67.5) (width 1.016) (layer "F.Cu") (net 37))
 (segment (start 115.9625 74) (end 117.2 74) (width 1.016) (layer "F.Cu") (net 37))
 (segment (start 145.25 66.15) (end 145.25 64.65) (width 1.016) (layer "F.Cu") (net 37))
 (segment (start 147.2 67.5) (end 145.85 66.15) (width 1.016) (layer "F.Cu") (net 37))
 (segment (start 143.9625 74.4) (end 146.6 71.7625) (width 1.016) (layer "F.Cu") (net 37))
 (segment (start 115.39 68.875) (end 115.39 63.95) (width 1.016) (layer "F.Cu") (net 37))
 (segment (start 146.6 71.7625) (end 147.2 71.1625) (width 1.016) (layer "F.Cu") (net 37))
 (segment (start 115.39 63.95) (end 117.57 61.77) (width 1.016) (layer "F.Cu") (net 37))
 (segment (start 145.85 66.15) (end 145.25 66.15) (width 1.016) (layer "F.Cu") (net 37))
 (segment (start 145.25 64.65) (end 143.55 62.95) (width 1.016) (layer "F.Cu") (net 37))
 (via (at 118.7 72.5) (size 0.8) (drill 0.4) (layers "F.Cu" "B.Cu") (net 37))
 (via (at 143.55 62.95) (size 1.397) (drill 1.016) (layers "F.Cu" "B.Cu") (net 37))
 (segment (start 115.39 68.875) (end 118.225 68.875) (width 1.016) (layer "B.Cu") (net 37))
 (segment (start 115.39 68.875) (end 115.39 69.19) (width 1.016) (layer "B.Cu") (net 37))
 (segment (start 143.5 62.9) (end 143.55 62.95) (width 0.25) (layer "B.Cu") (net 37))
 (segment (start 124.2 62.9) (end 143.5 62.9) (width 1.016) (layer "B.Cu") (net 37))
 (segment (start 115.39 69.19) (end 118.7 72.5) (width 1.016) (layer "B.Cu") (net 37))
 (segment (start 118.225 68.875) (end 124.2 62.9) (width 1.016) (layer "B.Cu") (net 37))
 (segment (start 136 60.4) (end 139 57.4) (width 0.635) (layer "F.Cu") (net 35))
 (segment (start 136 67.1) (end 142.75 67.1) (width 0.635) (layer "F.Cu") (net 35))
 (segment (start 136 67.1) (end 136 60.4) (width 0.635) (layer "F.Cu") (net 35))
 (segment (start 103 55.14) (end 103 54.2) (width 0.25) (layer "F.Cu") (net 45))
 (segment (start 106.76 58.9) (end 103 55.14) (width 0.25) (layer "F.Cu") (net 45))
 (segment (start 106.76 58.9) (end 109.63 61.77) (width 0.25) (layer "F.Cu") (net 45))
 (segment (start 103 58.9) (end 106.76 58.9) (width 0.25) (layer "F.Cu") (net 45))
 (segment (start 142.75 66.15) (end 142.75 65.05) (width 0.25) (layer "F.Cu") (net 34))
 (segment (start 142.75 65.05) (end 139 61.3) (width 0.25) (layer "F.Cu") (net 34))
 (via (at 139 61.3) (size 0.8) (drill 0.4) (layers "F.Cu" "B.Cu") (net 34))
 (segment (start 139 61.3) (end 128.7 61.3) (width 0.25) (layer "B.Cu") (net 34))
 (segment (start 100.38 61.82) (end 87.1 61.82) (width 0.25) (layer "B.Cu") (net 34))
 (segment (start 128.7 61.3) (end 121.4 54) (width 0.25) (layer "B.Cu") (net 34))
 (segment (start 108.2 54) (end 100.38 61.82) (width 0.25) (layer "B.Cu") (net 34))
 (segment (start 121.4 54) (end 108.2 54) (width 0.25) (layer "B.Cu") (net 34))
 (segment (start 145.25 70.65) (end 145.2 70.7) (width 0.25) (layer "F.Cu") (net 36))
 (segment (start 145.25 68.05) (end 145.25 70.65) (width 0.635) (layer "F.Cu") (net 36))
 (via (at 145.2 70.7) (size 1.016) (drill 0.635) (layers "F.Cu" "B.Cu") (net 36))
 (segment (start 145.1 70.6) (end 145.1 57.4) (width 0.635) (layer "B.Cu") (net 36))
 (segment (start 145.2 70.7) (end 145.1 70.6) (width 0.25) (layer "B.Cu") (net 36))
 (segment (start 92.1 110) (end 87.1 105) (width 1.016) (layer "F.Cu") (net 23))
 (segment (start 122.875 98.75) (end 132.915 98.75) (width 1.016) (layer "F.Cu") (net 23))
 (segment (start 121.95 98.75) (end 110.7 110) (width 1.016) (layer "F.Cu") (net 23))
 (segment (start 122.875 98.75) (end 121.95 98.75) (width 1.016) (layer "F.Cu") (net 23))
 (segment (start 77.06 55.9) (end 77.06 52.94) (width 0.25) (layer "F.Cu") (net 23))
 (segment (start 69.8 72.1) (end 69.8 87.7) (width 0.25) (layer "F.Cu") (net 23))
 (segment (start 110.7 110) (end 92.1 110) (width 1.016) (layer "F.Cu") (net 23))
 (segment (start 69.8 87.7) (end 87.1 105) (width 0.25) (layer "F.Cu") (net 23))
 (via (at 77.06 52.94) (size 0.8) (drill 0.4) (layers "F.Cu" "B.Cu") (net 23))
 (via (at 69.8 72.1) (size 0.8) (drill 0.4) (layers "F.Cu" "B.Cu") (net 23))
 (segment (start 69.8 60.2) (end 69.8 72.1) (width 0.25) (layer "B.Cu") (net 23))
 (segment (start 77.06 52.94) (end 69.8 60.2) (width 0.25) (layer "B.Cu") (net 23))
 (segment (start 124.1 84.46) (end 97.04 84.46) (width 0.25) (layer "F.Cu") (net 32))
 (segment (start 97.04 84.46) (end 87.1 74.52) (width 0.25) (layer "F.Cu") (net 32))
 (segment (start 125.8 77.7) (end 127.4 79.3) (width 0.25) (layer "B.Cu") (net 31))
 (segment (start 127.4 85.5) (end 125.9 87) (width 0.25) (layer "B.Cu") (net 31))
 (segment (start 127.4 79.3) (end 127.4 85.5) (width 0.25) (layer "B.Cu") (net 31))
 (segment (start 100.9 77.7) (end 125.8 77.7) (width 0.25) (layer "B.Cu") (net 31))
 (segment (start 125.9 87) (end 124.1 87) (width 0.25) (layer "B.Cu") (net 31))
 (segment (start 95.18 71.98) (end 100.9 77.7) (width 0.25) (layer "B.Cu") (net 31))
 (segment (start 87.1 71.98) (end 95.18 71.98) (width 0.25) (layer "B.Cu") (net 31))
 (segment (start 110.264956 102.764956) (end 110.264956 105.7) (width 0.25) (layer "F.Cu") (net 44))
 (segment (start 87.1 79.6) (end 110.264956 102.764956) (width 0.25) (layer "F.Cu") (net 44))
 (segment (start 87.1 82.14) (end 107.724956 102.764956) (width 0.25) (layer "F.Cu") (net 43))
 (segment (start 107.724956 102.764956) (end 107.724956 105.7) (width 0.25) (layer "F.Cu") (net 43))
 (segment (start 124.1 81.92) (end 91.96 81.92) (width 0.25) (layer "B.Cu") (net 33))
 (segment (start 91.96 81.92) (end 87.1 77.06) (width 0.25) (layer "B.Cu") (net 33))
 (segment (start 102.065 64.36) (end 103.625 62.8) (width 0.25) (layer "B.Cu") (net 40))
 (segment (start 87.1 64.36) (end 102.065 64.36) (width 0.25) (layer "B.Cu") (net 40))
 (segment (start 87.1 66.9) (end 102.065 66.9) (width 0.25) (layer "B.Cu") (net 41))
 (segment (start 102.065 66.9) (end 106.165 62.8) (width 0.25) (layer "B.Cu") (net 41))
 (segment (start 87.1 84.68) (end 94.52 92.1) (width 0.25) (layer "B.Cu") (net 30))
 (segment (start 94.52 92.1) (end 132.9 92.1) (width 0.25) (layer "B.Cu") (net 30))
 (segment (start 105.773 74.05) (end 91.71 74.05) (width 0.25) (layer "F.Cu") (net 1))
 (segment (start 91.71 74.05) (end 87.1 69.44) (width 0.25) (layer "F.Cu") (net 1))
 (segment (start 92.8 54.8) (end 91.85 53.85) (width 0.25) (layer "F.Cu") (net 3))
 (segment (start 90.6 52.6) (end 91.85 53.85) (width 0.25) (layer "F.Cu") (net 3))
 (segment (start 92.2 54.2) (end 92.3 54.2) (width 0.25) (layer "F.Cu") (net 3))
 (segment (start 92.8 56.7) (end 92.8 54.8) (width 0.25) (layer "F.Cu") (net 3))
 (segment (start 91.85 53.85) (end 92.2 54.2) (width 0.25) (layer "F.Cu") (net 3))
 (segment (start 92.3 54.2) (end 95.8625 54.2) (width 0.25) (layer "F.Cu") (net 3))
 (via (at 90.6 52.6) (size 0.8) (drill 0.4) (layers "F.Cu" "B.Cu") (free) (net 3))
 (segment (start 75.8 51.3) (end 89.3 51.3) (width 0.25) (layer "B.Cu") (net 3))
 (segment (start 64.24 54.2) (end 72.9 54.2) (width 0.25) (layer "B.Cu") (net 3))
 (segment (start 72.9 54.2) (end 75.8 51.3) (width 0.25) (layer "B.Cu") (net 3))
 (segment (start 89.3 51.3) (end 90.6 52.6) (width 0.25) (layer "B.Cu") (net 3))
 (segment (start 64.24 56.74) (end 66.28 54.7) (width 0.25) (layer "F.Cu") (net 4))
 (segment (start 66.28 54.7) (end 74.16 54.7) (width 0.25) (layer "F.Cu") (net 4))
 (segment (start 74.16 54.7) (end 74.86 55.4) (width 0.25) (layer "F.Cu") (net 4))
 (segment (start 74.86 55.4) (end 74.86 56.5) (width 0.25) (layer "F.Cu") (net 4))
 (segment (start 75.96 57.2) (end 75.96 56.1) (width 0.25) (layer "F.Cu") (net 5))
 (segment (start 64.24 59.28) (end 73.88 59.28) (width 0.25) (layer "F.Cu") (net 5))
 (segment (start 73.88 59.28) (end 75.96 57.2) (width 0.25) (layer "F.Cu") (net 5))
 (segment (start 64.24 61.82) (end 72.94 61.82) (width 0.25) (layer "F.Cu") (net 6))
 (segment (start 72.94 61.82) (end 78.16 56.6) (width 0.25) (layer "F.Cu") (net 6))
 (segment (start 78.16 56.6) (end 78.16 56.1) (width 0.25) (layer "F.Cu") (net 6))
 (segment (start 72.6 64.36) (end 80.36 56.6) (width 0.25) (layer "F.Cu") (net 7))
 (segment (start 64.24 64.36) (end 72.6 64.36) (width 0.25) (layer "F.Cu") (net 7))
 (segment (start 80.36 56.6) (end 80.36 56.1) (width 0.25) (layer "F.Cu") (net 7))
 (segment (start 95.4825 59.28) (end 95.8625 58.9) (width 0.25) (layer "F.Cu") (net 52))
 (segment (start 87.1 59.28) (end 95.4825 59.28) (width 0.25) (layer "F.Cu") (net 52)))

